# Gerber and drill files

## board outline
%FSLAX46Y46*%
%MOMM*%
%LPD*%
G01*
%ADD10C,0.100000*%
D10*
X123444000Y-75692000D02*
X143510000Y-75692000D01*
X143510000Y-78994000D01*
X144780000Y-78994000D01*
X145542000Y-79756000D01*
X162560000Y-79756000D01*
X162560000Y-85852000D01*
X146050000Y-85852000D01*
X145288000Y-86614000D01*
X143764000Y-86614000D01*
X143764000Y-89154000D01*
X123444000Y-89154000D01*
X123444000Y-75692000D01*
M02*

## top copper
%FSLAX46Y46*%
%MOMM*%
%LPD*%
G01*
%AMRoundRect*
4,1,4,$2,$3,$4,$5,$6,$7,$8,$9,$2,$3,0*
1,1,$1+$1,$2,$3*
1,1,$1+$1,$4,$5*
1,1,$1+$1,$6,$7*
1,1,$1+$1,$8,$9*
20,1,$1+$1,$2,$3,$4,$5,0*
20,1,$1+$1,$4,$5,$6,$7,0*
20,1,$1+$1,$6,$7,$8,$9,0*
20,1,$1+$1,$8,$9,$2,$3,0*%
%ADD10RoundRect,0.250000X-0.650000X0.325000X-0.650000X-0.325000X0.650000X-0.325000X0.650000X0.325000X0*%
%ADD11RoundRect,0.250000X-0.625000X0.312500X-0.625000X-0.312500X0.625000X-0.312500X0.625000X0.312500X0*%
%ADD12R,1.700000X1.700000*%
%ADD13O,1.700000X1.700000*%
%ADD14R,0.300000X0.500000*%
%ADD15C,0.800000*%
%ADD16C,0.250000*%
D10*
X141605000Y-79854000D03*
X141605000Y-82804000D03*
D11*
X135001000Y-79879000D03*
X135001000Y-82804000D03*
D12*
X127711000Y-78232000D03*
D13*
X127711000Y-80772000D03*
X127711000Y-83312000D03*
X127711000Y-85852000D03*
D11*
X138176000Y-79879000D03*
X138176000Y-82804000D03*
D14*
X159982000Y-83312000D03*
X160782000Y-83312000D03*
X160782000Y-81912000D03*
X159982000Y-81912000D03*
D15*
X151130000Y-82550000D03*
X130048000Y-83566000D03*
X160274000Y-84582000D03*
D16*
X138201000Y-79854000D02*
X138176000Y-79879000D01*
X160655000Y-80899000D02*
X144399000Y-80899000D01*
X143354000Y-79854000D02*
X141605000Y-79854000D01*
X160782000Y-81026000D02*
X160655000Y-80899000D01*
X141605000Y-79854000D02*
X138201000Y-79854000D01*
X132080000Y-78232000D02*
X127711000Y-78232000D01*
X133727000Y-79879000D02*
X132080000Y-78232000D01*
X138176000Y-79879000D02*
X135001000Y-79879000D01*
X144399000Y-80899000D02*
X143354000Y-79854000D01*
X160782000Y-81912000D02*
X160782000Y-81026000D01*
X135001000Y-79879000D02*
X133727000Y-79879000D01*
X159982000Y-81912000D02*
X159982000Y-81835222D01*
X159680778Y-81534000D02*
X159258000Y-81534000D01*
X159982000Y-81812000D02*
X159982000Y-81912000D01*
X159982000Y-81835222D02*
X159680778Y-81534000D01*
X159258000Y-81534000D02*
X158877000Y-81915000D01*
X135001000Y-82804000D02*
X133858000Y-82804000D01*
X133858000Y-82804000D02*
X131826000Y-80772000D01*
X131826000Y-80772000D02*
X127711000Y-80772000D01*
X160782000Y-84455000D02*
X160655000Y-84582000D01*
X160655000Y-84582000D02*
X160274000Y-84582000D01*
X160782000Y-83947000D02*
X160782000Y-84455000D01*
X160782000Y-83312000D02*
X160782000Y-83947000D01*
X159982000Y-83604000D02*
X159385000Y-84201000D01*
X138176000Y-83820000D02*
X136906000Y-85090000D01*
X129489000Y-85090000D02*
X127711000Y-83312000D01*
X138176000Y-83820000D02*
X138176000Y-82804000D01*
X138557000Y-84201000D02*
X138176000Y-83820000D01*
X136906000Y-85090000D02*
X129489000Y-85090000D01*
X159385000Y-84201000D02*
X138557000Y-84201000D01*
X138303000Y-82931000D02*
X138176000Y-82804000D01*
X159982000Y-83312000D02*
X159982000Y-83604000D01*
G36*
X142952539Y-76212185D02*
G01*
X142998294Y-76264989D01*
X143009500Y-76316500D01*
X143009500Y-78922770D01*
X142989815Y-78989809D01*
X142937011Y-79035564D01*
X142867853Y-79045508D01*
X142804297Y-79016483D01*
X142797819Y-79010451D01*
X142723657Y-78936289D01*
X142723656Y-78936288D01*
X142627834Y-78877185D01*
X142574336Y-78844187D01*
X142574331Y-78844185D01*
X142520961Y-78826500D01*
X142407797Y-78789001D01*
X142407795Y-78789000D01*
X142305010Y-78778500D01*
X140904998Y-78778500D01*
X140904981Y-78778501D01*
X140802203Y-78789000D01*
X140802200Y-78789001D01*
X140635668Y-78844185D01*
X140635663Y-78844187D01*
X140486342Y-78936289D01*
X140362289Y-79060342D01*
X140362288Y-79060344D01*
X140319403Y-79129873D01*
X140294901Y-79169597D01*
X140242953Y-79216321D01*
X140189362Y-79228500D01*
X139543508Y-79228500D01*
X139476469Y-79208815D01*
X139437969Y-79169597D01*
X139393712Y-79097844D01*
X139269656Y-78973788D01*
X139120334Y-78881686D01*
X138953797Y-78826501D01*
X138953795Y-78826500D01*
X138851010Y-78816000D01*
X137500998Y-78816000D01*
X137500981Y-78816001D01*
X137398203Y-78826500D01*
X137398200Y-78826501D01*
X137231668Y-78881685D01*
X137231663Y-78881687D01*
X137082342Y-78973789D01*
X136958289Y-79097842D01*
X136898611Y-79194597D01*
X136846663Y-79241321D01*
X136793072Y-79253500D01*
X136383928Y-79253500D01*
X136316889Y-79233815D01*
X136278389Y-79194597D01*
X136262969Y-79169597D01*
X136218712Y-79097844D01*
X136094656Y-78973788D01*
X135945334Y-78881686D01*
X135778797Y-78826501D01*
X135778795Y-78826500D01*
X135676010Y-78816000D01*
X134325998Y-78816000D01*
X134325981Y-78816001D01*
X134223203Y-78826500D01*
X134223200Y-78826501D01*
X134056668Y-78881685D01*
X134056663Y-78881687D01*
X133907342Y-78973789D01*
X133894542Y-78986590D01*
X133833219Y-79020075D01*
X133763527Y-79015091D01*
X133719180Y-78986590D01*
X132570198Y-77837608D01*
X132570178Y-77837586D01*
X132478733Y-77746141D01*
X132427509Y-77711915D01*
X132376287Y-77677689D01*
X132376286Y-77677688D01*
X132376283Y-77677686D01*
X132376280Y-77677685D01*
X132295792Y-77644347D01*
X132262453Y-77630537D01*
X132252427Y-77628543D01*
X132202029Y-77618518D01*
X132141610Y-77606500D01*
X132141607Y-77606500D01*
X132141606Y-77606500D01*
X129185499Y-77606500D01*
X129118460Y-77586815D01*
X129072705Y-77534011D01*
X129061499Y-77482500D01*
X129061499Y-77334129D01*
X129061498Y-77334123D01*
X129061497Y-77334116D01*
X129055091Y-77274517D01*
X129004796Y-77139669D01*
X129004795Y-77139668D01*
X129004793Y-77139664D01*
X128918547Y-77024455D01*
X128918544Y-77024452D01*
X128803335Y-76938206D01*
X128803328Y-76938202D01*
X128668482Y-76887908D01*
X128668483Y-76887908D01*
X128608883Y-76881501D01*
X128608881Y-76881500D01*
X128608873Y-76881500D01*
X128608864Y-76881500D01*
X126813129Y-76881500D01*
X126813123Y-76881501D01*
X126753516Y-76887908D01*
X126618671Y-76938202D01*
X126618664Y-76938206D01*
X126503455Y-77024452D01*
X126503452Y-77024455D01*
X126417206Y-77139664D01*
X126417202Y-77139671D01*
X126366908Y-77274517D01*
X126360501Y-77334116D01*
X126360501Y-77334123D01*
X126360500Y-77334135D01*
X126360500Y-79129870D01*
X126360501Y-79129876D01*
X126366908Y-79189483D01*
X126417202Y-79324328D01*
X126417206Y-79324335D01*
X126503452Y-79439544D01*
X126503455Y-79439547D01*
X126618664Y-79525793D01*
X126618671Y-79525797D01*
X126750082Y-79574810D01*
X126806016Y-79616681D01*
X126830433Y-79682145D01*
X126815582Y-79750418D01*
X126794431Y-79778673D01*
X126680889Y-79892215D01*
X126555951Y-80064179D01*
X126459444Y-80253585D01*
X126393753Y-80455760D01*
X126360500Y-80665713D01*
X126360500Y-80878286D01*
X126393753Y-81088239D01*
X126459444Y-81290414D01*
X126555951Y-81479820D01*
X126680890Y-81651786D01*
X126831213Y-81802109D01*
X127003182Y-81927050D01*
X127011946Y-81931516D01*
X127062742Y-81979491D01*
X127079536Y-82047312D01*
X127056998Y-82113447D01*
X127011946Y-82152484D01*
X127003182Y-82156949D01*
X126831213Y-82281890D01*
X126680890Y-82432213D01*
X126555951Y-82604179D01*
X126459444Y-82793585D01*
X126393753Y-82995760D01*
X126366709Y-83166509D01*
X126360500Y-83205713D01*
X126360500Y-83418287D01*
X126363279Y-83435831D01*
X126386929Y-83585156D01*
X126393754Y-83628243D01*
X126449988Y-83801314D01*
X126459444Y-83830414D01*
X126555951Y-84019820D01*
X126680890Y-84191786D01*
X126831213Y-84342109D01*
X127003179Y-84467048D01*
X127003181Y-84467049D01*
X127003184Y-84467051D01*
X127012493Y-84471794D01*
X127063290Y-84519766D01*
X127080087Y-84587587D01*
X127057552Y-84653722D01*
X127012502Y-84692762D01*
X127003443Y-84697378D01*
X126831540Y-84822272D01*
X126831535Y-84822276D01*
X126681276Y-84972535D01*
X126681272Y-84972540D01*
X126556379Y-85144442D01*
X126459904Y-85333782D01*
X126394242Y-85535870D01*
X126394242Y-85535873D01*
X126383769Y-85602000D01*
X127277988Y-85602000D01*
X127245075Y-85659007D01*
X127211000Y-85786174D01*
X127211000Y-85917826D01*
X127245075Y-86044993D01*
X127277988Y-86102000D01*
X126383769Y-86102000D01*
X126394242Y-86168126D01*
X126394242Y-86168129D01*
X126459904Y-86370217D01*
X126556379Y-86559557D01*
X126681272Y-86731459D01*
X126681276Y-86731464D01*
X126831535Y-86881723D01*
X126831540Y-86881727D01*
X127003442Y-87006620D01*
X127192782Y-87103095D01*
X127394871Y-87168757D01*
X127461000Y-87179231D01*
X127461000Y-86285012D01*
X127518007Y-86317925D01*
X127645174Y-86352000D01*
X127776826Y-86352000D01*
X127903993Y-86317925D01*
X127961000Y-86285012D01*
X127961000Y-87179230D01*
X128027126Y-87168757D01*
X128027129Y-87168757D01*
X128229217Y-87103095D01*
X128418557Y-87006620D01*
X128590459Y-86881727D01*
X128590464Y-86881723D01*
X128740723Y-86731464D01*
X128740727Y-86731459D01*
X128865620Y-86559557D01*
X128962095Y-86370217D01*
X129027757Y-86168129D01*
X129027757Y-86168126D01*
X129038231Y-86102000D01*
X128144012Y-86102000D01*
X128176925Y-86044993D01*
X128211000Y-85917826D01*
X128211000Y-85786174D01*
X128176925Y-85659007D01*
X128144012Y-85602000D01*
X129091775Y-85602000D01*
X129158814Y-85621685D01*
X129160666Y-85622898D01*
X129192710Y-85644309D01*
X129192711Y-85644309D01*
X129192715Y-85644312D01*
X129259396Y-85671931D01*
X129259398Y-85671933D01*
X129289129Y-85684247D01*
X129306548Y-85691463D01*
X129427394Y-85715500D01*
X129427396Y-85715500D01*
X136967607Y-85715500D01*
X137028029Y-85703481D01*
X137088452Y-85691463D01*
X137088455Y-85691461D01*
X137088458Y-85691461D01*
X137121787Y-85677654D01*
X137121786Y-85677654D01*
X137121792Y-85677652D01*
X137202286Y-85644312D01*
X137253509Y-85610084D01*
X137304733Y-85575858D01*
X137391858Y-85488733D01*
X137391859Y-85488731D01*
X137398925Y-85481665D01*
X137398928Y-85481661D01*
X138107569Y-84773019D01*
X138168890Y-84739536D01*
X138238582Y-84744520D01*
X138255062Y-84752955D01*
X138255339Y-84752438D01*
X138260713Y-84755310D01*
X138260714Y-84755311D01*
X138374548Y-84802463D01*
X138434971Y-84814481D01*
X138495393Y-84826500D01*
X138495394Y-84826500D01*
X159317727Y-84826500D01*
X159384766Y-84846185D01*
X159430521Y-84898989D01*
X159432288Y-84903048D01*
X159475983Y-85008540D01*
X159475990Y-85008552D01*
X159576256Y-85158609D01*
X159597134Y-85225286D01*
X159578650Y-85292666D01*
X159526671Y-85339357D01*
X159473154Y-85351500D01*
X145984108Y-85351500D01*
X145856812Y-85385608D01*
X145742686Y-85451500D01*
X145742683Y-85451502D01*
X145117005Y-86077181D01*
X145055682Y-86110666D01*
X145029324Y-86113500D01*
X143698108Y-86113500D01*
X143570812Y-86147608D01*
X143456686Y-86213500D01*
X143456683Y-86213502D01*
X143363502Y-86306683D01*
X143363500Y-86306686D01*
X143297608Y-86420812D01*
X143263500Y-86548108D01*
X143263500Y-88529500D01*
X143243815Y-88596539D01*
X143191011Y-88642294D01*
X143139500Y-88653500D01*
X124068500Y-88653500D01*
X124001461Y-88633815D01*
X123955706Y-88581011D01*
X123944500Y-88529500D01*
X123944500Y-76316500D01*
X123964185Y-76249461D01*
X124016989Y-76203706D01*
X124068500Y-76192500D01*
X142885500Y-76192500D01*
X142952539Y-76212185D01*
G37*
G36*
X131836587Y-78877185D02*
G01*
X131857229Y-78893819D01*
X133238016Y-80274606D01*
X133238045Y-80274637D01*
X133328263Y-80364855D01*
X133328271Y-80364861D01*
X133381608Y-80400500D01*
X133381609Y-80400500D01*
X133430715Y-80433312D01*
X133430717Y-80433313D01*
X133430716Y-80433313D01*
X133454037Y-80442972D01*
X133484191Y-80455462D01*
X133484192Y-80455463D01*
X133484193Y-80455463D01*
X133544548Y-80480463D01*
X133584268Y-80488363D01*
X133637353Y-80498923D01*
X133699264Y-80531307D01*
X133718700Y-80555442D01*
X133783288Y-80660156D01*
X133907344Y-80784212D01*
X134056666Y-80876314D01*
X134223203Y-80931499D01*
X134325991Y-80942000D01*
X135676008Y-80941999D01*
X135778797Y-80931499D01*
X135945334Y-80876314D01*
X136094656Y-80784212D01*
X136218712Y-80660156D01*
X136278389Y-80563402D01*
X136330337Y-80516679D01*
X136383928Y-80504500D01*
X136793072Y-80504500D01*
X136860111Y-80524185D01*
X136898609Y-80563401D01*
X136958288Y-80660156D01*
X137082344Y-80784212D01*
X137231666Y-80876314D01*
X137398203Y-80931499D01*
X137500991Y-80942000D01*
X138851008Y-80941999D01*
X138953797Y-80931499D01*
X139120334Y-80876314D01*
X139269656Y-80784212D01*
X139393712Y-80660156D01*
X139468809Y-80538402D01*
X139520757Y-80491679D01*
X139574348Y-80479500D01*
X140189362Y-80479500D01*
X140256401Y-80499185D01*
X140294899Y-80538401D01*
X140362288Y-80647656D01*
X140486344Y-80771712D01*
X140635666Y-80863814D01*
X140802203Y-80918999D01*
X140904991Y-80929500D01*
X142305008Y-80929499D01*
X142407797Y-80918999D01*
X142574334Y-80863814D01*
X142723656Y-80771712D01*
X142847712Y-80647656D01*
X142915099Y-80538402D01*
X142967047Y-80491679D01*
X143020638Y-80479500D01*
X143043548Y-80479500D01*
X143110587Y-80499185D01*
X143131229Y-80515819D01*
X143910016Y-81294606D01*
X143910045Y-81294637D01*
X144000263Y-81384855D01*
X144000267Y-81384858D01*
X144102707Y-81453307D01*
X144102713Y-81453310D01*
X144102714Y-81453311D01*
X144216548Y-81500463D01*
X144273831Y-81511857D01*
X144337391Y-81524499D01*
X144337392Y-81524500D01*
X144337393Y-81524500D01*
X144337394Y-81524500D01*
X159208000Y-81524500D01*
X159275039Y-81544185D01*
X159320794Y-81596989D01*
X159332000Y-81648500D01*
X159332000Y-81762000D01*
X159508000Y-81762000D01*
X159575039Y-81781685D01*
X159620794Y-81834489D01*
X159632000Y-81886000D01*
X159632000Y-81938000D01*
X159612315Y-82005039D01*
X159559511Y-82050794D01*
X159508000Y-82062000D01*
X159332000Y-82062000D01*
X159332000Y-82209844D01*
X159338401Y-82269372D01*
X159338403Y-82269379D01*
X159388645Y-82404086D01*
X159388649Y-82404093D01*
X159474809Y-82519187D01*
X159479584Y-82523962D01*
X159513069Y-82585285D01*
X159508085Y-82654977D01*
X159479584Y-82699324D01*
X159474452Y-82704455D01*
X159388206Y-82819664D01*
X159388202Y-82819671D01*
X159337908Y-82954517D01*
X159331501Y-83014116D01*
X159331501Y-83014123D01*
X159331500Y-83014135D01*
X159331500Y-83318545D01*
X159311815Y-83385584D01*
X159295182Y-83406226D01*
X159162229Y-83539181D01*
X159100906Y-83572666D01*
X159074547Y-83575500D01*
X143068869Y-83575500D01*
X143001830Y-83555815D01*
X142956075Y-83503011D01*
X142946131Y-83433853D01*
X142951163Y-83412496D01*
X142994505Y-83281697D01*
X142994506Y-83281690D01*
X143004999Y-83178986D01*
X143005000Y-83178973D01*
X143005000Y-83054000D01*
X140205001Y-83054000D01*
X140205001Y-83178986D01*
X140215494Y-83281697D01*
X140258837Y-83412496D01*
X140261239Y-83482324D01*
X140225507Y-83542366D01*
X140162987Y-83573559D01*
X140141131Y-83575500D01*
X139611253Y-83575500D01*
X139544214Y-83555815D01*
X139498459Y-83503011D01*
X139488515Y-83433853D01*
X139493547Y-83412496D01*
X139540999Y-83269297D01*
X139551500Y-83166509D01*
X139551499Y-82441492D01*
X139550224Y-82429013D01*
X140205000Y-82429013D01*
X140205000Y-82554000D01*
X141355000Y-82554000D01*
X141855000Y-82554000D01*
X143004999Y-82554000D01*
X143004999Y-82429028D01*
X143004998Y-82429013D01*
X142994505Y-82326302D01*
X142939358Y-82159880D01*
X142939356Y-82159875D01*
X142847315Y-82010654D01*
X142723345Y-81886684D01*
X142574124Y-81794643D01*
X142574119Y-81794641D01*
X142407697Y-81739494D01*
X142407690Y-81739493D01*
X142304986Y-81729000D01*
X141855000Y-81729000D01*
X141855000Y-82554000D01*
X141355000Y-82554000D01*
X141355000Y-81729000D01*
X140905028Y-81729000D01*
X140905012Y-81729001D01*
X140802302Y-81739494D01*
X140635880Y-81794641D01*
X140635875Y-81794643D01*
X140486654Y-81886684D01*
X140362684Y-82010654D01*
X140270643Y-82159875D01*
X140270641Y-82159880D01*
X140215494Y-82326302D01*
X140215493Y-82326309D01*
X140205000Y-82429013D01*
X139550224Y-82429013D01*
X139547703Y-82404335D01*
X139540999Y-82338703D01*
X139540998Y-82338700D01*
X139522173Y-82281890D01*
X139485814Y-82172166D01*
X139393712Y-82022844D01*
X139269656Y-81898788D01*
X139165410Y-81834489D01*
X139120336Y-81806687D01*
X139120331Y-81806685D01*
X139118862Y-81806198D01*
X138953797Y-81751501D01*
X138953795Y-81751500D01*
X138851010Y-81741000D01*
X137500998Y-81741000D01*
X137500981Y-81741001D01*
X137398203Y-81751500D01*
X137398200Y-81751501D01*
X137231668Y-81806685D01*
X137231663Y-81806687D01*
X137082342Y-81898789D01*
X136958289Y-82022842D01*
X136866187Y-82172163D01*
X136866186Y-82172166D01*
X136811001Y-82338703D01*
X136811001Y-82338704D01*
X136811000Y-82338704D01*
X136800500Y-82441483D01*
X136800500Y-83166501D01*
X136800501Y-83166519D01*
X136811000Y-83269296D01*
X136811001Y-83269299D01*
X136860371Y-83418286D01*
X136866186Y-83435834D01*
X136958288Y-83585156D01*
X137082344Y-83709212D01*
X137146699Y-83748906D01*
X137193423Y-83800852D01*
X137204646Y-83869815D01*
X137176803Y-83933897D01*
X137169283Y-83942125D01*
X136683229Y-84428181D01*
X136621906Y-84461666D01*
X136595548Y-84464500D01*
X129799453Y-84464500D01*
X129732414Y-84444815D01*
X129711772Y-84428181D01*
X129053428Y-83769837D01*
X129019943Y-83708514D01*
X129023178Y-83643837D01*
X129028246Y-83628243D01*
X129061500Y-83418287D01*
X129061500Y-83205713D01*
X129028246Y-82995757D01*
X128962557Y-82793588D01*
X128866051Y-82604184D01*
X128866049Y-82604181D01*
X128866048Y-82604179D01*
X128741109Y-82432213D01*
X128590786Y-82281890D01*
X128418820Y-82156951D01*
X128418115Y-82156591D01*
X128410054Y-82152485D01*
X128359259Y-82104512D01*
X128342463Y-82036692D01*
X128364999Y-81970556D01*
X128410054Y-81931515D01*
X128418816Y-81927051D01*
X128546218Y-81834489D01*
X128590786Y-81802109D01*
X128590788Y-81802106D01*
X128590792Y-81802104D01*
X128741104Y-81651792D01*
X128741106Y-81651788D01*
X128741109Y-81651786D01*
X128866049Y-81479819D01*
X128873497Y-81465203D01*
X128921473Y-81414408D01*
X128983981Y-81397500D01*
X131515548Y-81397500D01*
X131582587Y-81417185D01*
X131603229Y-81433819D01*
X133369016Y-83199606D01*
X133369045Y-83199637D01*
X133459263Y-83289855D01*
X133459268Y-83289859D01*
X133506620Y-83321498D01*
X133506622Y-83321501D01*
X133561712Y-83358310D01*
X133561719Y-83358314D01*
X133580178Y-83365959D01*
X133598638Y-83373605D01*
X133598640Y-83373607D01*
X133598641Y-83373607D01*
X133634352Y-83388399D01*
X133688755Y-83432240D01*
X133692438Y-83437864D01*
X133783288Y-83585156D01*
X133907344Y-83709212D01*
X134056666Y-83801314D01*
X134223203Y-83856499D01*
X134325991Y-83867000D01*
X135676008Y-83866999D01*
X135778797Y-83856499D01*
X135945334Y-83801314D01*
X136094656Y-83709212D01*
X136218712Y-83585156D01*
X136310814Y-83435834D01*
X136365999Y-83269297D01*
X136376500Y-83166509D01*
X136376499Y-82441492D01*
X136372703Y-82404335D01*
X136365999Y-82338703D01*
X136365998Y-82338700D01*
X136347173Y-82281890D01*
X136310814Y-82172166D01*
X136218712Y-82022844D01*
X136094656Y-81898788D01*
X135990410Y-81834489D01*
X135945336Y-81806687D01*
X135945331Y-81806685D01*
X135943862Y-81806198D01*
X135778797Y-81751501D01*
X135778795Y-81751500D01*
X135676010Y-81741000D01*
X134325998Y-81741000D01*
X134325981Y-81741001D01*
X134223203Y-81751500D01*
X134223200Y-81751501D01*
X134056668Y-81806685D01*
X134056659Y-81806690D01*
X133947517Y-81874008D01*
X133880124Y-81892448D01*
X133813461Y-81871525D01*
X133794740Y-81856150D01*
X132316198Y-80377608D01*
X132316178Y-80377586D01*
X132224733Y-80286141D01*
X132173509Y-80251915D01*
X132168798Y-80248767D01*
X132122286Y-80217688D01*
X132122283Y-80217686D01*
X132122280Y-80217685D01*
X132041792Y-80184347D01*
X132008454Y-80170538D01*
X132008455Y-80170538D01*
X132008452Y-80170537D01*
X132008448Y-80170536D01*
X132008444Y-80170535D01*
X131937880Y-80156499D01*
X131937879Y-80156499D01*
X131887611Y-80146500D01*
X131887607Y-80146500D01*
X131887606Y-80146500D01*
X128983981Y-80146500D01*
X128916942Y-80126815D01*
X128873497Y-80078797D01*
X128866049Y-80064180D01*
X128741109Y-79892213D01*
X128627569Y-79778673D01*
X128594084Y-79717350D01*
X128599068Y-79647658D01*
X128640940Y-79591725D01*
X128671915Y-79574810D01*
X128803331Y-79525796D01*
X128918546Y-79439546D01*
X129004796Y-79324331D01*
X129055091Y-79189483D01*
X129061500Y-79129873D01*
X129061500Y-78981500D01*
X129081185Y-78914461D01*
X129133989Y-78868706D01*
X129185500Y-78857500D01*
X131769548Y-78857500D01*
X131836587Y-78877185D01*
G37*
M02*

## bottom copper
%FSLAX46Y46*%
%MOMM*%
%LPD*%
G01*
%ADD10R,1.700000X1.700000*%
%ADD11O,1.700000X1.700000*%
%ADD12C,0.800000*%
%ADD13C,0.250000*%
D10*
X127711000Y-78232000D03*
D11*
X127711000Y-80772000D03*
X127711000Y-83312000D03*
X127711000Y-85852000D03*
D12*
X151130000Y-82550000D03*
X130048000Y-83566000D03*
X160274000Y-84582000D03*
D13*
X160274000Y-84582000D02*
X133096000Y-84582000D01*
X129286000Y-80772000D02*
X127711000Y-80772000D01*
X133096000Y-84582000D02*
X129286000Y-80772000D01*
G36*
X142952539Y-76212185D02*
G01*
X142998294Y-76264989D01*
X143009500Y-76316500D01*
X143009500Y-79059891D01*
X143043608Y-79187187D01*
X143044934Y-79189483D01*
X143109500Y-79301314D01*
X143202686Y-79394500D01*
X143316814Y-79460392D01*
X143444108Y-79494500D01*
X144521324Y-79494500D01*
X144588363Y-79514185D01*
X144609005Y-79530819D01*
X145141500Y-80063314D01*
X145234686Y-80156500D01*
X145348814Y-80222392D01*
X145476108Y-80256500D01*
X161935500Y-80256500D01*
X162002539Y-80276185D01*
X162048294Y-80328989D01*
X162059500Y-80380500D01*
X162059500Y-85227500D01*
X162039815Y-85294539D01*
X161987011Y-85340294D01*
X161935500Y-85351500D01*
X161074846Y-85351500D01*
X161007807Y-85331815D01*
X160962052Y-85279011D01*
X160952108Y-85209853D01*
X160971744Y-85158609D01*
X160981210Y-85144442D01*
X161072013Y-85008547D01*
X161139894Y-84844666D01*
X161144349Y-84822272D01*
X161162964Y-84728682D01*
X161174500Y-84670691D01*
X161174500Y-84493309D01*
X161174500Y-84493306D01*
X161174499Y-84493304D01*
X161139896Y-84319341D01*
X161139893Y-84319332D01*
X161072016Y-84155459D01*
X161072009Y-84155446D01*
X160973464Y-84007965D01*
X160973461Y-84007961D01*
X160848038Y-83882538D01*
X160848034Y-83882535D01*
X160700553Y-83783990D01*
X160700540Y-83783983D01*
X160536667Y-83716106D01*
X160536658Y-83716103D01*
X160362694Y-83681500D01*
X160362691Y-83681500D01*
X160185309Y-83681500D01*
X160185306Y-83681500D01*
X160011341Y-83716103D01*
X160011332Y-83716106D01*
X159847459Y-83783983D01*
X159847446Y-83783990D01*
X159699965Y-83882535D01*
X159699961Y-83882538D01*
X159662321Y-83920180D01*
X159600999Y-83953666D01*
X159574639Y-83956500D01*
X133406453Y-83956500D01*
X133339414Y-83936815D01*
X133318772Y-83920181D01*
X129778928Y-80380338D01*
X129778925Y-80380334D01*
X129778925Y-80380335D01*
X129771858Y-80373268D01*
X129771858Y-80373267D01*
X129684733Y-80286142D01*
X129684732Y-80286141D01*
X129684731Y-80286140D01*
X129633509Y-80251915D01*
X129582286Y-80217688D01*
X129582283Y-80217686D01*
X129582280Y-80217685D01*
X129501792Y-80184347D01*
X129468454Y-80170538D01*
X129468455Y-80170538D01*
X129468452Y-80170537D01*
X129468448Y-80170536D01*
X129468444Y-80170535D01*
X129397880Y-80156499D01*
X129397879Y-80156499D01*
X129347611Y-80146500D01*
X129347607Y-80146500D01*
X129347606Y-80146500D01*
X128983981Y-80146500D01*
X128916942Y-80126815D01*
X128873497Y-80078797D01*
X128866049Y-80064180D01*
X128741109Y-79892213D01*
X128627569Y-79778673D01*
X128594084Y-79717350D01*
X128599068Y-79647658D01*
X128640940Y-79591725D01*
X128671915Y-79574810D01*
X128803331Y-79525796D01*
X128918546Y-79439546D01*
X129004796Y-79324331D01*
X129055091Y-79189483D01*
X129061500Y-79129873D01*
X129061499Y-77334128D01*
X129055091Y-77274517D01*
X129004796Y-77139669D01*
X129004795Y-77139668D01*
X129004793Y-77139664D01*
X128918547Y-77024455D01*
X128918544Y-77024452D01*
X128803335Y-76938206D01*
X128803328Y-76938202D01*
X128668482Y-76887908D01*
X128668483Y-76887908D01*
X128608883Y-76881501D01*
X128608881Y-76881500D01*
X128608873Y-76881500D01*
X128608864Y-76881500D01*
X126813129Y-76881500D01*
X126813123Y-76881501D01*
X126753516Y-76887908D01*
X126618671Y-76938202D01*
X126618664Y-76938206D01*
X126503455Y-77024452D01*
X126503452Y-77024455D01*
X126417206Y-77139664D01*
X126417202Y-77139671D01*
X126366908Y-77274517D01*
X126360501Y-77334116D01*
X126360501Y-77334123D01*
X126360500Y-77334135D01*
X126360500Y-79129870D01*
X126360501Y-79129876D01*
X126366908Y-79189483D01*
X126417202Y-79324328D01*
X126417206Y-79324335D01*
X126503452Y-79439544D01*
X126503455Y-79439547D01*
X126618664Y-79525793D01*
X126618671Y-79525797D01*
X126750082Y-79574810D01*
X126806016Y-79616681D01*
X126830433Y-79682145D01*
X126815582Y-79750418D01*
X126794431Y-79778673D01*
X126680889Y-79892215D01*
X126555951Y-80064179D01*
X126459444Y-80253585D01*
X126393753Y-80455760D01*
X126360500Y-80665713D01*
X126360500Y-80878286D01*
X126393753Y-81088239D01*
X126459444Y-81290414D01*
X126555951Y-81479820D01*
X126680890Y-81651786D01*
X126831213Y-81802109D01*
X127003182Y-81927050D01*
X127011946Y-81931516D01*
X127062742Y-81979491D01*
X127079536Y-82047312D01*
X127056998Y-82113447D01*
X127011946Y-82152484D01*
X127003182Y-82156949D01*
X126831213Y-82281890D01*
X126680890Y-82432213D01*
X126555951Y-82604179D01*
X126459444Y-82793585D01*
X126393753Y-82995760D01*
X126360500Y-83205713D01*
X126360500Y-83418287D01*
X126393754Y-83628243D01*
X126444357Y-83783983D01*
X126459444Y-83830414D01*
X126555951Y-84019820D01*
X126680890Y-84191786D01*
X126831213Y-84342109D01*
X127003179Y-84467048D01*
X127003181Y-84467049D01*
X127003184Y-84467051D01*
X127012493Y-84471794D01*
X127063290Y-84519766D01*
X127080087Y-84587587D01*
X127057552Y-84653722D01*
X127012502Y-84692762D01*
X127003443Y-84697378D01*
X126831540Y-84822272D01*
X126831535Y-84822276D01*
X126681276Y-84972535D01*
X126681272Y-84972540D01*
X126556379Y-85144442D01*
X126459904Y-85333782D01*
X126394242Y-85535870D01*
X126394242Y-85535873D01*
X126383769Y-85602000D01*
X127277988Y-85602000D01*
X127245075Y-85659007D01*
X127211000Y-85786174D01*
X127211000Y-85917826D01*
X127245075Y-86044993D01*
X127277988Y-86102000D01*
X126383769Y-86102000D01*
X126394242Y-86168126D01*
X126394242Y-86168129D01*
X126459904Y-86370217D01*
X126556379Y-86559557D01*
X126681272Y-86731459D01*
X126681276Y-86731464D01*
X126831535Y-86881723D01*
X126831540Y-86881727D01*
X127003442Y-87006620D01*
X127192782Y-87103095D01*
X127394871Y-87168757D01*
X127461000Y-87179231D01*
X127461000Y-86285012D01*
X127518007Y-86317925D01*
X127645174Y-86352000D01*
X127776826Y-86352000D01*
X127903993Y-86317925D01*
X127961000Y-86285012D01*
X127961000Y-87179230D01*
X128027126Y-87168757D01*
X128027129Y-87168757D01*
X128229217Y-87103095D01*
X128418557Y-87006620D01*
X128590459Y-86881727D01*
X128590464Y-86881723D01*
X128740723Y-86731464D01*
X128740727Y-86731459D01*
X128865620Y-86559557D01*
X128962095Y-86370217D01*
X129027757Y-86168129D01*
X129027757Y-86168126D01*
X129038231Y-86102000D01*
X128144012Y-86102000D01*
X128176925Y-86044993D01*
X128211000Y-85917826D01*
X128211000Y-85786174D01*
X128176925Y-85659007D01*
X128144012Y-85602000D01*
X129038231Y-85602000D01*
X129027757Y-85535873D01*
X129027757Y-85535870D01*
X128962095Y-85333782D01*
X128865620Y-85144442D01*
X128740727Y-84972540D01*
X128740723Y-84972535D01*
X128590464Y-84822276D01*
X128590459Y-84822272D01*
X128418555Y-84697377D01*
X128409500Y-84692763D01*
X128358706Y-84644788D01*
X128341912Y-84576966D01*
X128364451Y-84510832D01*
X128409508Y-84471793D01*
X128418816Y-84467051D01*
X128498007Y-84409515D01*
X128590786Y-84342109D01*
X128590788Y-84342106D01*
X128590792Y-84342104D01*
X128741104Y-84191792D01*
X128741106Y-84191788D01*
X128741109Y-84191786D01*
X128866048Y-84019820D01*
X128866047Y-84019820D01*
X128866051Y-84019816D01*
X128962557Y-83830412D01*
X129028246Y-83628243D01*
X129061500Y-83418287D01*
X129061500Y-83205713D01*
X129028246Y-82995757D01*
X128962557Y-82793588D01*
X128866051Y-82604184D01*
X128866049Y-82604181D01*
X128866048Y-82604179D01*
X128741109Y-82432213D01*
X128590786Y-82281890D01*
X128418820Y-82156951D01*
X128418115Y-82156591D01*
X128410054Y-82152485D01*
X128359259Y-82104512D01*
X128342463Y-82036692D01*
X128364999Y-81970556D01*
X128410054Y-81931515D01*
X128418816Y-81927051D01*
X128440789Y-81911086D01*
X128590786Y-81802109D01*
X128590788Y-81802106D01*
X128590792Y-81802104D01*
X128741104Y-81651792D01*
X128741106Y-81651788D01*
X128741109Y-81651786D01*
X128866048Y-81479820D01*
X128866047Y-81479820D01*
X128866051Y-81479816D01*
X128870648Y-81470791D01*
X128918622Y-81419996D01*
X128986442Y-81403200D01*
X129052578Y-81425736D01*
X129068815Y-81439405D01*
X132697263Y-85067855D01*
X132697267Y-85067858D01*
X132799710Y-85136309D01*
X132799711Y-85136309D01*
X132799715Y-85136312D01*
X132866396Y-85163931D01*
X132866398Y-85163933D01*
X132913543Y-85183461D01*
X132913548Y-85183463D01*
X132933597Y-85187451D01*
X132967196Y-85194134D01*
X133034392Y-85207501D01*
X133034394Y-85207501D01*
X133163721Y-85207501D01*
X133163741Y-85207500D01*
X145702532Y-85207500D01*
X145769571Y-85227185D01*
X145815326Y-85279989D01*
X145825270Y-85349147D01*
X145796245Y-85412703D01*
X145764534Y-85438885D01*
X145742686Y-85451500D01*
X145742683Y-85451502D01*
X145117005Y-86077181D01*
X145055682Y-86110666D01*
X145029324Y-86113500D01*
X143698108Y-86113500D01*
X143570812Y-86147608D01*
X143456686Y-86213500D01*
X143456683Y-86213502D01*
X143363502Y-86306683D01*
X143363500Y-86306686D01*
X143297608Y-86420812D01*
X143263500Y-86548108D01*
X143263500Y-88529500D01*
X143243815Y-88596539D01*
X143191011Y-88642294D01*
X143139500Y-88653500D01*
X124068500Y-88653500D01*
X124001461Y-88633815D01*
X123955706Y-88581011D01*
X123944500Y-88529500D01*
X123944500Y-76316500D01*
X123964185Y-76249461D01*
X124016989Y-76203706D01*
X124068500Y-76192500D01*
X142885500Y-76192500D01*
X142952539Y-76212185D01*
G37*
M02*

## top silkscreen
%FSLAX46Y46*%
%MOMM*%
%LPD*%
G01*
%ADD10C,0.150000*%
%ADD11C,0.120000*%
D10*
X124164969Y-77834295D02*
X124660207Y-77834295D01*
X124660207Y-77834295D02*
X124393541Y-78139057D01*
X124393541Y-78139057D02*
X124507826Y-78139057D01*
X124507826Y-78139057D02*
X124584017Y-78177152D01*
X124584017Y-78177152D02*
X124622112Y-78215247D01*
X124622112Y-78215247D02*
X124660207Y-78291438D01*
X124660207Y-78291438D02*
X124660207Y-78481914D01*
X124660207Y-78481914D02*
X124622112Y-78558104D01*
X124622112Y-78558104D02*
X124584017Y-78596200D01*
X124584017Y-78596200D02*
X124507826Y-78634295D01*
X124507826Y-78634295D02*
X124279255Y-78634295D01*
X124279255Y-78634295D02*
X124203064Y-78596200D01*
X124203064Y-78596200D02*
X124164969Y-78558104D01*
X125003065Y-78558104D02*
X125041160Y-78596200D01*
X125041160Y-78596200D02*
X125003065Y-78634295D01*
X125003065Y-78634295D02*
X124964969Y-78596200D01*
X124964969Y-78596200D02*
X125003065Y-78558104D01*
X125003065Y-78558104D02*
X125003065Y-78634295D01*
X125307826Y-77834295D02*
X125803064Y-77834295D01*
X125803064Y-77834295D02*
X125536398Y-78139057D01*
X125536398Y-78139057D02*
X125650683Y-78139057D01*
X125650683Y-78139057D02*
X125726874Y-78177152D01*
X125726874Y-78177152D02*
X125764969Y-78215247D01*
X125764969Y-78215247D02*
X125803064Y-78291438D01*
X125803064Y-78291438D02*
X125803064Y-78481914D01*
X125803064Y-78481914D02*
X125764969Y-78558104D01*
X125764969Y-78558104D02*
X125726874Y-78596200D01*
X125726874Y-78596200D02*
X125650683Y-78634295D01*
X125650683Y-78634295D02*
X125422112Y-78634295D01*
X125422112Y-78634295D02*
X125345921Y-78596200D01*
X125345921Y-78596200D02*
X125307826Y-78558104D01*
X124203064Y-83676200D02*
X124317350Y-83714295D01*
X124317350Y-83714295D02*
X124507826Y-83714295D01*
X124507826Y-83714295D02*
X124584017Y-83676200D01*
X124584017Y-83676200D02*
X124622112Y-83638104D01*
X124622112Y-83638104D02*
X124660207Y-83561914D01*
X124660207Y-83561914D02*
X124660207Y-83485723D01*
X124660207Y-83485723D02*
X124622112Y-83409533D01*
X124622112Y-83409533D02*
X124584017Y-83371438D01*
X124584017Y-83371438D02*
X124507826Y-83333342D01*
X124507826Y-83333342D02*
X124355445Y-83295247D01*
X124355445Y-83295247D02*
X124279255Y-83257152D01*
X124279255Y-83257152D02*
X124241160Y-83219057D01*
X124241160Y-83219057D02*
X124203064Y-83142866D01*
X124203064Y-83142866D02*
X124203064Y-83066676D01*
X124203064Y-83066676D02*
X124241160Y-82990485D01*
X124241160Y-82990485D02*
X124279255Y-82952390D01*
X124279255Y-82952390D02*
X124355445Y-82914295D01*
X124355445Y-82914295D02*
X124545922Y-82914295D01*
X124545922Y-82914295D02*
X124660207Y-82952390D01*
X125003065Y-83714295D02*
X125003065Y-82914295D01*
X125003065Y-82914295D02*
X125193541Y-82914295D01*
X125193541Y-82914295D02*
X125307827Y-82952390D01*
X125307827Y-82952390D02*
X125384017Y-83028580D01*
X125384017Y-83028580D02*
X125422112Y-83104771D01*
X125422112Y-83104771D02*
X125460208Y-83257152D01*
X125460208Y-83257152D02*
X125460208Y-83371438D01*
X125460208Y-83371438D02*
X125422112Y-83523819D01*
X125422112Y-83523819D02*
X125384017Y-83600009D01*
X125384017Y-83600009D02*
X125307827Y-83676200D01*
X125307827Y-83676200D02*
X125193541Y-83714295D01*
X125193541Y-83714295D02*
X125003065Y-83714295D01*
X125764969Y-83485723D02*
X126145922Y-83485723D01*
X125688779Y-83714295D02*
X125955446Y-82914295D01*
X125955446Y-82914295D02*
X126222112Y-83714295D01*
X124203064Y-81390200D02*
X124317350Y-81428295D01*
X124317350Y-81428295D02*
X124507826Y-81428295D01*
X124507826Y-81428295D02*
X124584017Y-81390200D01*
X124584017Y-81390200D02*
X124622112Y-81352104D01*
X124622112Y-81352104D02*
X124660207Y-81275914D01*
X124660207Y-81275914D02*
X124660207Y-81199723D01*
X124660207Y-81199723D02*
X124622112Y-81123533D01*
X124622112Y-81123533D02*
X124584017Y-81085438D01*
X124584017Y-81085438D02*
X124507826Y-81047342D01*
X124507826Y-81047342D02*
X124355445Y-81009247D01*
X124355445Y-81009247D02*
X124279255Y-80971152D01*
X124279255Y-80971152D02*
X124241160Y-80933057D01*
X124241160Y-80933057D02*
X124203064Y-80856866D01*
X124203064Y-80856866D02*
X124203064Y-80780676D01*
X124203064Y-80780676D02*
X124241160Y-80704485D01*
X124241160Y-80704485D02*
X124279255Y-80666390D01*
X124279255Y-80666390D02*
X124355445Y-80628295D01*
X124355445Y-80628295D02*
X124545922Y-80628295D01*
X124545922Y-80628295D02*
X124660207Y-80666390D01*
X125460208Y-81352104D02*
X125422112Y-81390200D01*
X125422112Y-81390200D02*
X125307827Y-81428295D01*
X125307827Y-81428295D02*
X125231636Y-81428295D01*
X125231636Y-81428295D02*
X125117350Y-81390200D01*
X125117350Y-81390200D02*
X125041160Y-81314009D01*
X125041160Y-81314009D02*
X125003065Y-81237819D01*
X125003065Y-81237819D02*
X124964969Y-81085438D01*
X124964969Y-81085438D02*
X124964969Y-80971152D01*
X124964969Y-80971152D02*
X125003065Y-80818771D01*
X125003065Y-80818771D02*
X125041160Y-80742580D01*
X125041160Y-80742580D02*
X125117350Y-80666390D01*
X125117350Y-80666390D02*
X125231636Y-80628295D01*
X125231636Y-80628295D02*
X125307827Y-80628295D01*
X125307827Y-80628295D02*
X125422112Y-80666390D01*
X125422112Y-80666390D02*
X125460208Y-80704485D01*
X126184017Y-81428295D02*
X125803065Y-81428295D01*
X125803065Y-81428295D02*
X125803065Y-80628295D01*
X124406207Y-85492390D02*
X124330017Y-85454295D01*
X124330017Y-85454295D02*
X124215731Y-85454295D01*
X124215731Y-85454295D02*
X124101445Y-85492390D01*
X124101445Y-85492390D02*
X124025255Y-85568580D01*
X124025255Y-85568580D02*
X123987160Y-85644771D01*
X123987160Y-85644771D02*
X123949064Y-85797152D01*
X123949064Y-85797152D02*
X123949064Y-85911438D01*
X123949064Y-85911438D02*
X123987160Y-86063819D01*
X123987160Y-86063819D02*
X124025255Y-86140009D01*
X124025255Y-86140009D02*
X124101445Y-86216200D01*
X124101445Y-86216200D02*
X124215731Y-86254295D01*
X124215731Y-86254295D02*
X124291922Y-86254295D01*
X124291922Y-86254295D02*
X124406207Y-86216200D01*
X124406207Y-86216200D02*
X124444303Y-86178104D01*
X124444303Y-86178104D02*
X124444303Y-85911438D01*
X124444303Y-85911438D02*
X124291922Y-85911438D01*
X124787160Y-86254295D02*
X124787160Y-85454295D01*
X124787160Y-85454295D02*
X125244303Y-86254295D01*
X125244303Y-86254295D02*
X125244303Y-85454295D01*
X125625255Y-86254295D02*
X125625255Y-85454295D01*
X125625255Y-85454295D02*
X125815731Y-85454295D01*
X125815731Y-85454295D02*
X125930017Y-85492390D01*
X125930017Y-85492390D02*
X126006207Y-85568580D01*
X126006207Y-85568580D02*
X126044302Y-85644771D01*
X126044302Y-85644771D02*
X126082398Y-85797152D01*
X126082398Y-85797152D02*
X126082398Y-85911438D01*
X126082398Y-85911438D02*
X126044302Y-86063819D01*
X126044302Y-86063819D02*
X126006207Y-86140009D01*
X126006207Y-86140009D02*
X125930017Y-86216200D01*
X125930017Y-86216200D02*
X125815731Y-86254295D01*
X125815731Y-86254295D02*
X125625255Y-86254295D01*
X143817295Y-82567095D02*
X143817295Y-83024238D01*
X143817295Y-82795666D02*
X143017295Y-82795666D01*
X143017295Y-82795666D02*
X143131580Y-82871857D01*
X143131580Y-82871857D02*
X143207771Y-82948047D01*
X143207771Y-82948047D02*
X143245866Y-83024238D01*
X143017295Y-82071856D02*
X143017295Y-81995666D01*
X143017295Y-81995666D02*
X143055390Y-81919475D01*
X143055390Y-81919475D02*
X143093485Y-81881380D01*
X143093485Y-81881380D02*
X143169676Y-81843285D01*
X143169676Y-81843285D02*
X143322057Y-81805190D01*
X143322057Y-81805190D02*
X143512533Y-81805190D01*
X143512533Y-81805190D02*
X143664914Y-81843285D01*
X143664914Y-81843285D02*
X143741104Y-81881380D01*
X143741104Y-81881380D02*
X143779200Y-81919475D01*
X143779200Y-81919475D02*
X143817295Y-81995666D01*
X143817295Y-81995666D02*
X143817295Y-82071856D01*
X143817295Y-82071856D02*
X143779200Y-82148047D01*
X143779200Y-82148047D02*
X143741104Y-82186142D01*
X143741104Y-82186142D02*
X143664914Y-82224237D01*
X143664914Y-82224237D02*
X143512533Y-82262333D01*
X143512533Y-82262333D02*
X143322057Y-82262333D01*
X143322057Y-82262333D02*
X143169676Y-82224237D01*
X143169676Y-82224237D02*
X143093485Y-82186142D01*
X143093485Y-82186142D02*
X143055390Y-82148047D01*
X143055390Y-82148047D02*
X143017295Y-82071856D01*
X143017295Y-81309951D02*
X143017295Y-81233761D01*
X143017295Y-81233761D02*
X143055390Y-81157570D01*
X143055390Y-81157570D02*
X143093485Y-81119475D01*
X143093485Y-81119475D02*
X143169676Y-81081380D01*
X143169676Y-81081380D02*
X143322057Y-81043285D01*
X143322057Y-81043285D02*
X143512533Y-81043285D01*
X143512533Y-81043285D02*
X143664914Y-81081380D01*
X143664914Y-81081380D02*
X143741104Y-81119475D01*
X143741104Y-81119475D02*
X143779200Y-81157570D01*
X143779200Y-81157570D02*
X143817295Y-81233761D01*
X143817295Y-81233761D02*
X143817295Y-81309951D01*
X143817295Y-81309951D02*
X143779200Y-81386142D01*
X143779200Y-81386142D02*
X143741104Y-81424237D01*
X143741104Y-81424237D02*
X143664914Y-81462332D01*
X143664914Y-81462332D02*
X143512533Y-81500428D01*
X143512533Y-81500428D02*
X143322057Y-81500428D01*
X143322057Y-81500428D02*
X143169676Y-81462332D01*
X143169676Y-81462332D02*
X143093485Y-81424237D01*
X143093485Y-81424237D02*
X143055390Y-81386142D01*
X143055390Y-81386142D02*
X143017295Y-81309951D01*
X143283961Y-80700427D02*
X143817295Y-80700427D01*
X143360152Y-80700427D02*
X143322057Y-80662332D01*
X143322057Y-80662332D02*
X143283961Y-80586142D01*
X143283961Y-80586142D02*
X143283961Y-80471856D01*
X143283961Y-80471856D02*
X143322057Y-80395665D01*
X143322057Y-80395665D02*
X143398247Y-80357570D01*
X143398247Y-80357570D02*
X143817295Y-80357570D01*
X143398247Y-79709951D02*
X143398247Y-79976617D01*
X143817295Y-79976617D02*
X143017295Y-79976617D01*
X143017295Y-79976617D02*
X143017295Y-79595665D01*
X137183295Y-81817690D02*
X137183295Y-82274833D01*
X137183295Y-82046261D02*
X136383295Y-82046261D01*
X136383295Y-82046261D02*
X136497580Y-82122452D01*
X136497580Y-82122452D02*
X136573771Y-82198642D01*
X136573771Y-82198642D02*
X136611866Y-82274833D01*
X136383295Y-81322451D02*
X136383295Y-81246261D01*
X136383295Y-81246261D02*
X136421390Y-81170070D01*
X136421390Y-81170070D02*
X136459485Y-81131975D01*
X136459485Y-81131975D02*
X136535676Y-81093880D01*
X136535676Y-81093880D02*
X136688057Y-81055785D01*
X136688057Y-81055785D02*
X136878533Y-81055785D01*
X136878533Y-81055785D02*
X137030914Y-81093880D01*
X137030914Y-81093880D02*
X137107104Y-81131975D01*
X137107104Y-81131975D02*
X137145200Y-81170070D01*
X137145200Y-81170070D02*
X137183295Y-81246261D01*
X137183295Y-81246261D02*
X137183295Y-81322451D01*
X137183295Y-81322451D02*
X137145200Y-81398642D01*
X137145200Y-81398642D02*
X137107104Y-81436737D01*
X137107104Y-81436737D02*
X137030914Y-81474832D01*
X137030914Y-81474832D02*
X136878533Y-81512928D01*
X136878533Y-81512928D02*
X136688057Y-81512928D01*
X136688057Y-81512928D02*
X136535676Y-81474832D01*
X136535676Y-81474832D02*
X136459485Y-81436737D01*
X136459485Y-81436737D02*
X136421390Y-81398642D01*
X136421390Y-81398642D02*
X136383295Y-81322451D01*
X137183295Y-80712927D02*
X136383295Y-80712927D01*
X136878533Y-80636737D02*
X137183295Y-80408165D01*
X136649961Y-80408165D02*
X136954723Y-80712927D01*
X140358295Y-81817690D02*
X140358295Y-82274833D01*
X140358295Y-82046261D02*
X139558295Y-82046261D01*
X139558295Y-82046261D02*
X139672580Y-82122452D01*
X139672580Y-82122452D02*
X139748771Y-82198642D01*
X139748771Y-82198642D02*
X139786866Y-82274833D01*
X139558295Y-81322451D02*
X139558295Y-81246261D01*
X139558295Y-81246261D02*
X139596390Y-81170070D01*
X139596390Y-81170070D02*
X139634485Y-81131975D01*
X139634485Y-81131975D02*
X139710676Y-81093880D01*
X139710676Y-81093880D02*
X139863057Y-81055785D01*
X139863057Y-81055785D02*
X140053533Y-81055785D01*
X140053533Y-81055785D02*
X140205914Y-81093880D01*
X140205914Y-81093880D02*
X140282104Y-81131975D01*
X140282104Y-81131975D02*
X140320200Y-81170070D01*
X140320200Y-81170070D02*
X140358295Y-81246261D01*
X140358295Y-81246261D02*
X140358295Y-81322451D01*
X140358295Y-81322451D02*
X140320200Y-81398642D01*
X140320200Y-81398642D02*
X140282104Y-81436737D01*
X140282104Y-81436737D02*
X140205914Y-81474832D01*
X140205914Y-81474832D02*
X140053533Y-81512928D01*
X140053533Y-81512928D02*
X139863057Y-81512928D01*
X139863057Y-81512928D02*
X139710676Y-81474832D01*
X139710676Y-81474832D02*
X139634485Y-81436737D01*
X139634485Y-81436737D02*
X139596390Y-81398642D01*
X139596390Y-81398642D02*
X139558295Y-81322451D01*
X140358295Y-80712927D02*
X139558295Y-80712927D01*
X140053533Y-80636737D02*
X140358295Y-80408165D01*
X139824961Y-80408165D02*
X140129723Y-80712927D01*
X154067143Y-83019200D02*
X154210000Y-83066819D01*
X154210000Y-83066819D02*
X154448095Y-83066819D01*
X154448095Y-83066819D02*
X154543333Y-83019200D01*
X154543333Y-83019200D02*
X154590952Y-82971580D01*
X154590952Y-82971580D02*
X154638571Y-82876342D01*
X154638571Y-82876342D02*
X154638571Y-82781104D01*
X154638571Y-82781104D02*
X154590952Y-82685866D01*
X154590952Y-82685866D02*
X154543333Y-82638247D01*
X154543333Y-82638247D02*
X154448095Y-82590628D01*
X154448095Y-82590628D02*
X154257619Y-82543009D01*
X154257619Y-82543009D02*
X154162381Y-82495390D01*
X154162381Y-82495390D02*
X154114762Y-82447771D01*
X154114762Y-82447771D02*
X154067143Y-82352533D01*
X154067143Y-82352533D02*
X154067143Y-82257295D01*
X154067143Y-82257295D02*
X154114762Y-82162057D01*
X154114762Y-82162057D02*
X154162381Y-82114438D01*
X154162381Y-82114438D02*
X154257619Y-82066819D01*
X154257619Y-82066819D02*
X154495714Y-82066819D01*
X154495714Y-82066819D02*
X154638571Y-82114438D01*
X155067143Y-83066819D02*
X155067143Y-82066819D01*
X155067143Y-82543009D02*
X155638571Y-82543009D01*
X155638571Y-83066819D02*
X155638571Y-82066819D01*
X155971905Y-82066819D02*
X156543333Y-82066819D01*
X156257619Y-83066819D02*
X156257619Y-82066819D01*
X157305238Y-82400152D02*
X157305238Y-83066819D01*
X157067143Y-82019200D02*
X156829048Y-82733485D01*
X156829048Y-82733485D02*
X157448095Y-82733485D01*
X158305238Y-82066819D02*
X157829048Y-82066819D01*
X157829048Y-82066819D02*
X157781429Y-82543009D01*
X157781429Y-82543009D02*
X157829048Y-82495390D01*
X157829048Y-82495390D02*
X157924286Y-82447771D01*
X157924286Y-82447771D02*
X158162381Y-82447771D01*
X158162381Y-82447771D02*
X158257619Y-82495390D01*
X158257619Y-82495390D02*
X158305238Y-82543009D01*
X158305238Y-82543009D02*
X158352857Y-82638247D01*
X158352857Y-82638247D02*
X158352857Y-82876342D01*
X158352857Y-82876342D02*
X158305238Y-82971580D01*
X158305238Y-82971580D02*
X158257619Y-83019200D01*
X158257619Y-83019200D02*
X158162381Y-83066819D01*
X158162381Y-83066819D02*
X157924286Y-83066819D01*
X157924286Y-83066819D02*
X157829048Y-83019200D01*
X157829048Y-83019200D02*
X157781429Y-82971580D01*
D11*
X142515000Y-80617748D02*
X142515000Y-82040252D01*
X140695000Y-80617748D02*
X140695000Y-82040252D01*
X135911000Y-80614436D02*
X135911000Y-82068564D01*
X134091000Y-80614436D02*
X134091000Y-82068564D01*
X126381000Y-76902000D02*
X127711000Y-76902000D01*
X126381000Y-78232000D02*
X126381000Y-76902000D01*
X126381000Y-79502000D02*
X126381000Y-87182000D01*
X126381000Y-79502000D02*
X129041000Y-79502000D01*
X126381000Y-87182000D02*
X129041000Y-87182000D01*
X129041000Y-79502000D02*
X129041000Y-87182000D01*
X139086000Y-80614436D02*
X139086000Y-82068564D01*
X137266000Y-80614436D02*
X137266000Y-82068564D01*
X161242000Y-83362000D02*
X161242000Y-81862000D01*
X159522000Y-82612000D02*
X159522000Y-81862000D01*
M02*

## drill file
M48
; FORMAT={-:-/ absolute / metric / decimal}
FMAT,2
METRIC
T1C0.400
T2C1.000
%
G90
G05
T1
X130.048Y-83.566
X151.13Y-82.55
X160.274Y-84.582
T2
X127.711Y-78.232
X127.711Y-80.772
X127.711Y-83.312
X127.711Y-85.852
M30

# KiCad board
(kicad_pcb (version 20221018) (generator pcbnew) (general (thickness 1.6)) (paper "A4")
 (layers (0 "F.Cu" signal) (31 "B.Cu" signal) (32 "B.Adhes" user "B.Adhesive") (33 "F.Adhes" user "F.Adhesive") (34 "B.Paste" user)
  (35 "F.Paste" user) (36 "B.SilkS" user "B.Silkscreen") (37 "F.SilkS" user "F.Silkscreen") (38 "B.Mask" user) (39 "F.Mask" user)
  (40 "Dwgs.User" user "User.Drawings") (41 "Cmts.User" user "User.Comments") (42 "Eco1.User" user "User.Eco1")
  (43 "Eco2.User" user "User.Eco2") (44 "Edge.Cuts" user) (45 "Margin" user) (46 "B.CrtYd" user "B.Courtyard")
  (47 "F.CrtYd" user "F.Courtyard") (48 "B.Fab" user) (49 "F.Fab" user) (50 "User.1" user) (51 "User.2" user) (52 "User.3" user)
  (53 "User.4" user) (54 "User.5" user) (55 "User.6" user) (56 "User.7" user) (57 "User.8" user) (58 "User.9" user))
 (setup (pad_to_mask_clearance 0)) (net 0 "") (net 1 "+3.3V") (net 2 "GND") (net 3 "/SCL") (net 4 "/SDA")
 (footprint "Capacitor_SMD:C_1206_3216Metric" (layer "F.Cu") (at 141.605 81.329 -90)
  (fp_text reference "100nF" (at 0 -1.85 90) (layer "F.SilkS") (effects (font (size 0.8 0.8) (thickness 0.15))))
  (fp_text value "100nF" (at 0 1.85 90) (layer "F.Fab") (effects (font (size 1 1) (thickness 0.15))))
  (fp_line (start -0.711252 -0.91) (end 0.711252 -0.91) (stroke (width 0.12) (type solid)) (layer "F.SilkS"))
  (fp_line (start -0.711252 0.91) (end 0.711252 0.91) (stroke (width 0.12) (type solid)) (layer "F.SilkS"))
  (pad "1" smd roundrect (at -1.475 0 270) (size 1.15 1.8) (layers "F.Cu" "F.Paste" "F.Mask") (roundrect_rratio 0.2173913043)
   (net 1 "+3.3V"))
  (pad "2" smd roundrect (at 1.475 0 270) (size 1.15 1.8) (layers "F.Cu" "F.Paste" "F.Mask") (roundrect_rratio 0.2173913043) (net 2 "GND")))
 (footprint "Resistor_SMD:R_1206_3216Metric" (layer "F.Cu") (at 135.001 81.3415 -90)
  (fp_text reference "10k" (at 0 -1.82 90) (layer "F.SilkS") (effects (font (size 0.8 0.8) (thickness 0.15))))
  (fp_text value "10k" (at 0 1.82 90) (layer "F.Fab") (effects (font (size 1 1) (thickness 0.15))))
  (fp_line (start -0.727064 -0.91) (end 0.727064 -0.91) (stroke (width 0.12) (type solid)) (layer "F.SilkS"))
  (fp_line (start -0.727064 0.91) (end 0.727064 0.91) (stroke (width 0.12) (type solid)) (layer "F.SilkS"))
  (pad "1" smd roundrect (at -1.4625 0 270) (size 1.125 1.75) (layers "F.Cu" "F.Paste" "F.Mask") (roundrect_rratio 0.2222222222)
   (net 1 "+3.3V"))
  (pad "2" smd roundrect (at 1.4625 0 270) (size 1.125 1.75) (layers "F.Cu" "F.Paste" "F.Mask") (roundrect_rratio 0.2222222222)
   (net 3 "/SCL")))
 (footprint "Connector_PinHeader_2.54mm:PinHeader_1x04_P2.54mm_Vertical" (layer "F.Cu") (at 127.711 78.232)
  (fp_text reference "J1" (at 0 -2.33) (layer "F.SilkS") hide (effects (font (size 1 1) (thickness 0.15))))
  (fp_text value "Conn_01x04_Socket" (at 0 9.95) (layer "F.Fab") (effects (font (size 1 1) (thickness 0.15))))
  (fp_line (start -1.33 -1.33) (end 0 -1.33) (stroke (width 0.12) (type solid)) (layer "F.SilkS"))
  (fp_line (start -1.33 0) (end -1.33 -1.33) (stroke (width 0.12) (type solid)) (layer "F.SilkS"))
  (fp_line (start -1.33 1.27) (end -1.33 8.95) (stroke (width 0.12) (type solid)) (layer "F.SilkS"))
  (fp_line (start -1.33 1.27) (end 1.33 1.27) (stroke (width 0.12) (type solid)) (layer "F.SilkS"))
  (fp_line (start -1.33 8.95) (end 1.33 8.95) (stroke (width 0.12) (type solid)) (layer "F.SilkS"))
  (fp_line (start 1.33 1.27) (end 1.33 8.95) (stroke (width 0.12) (type solid)) (layer "F.SilkS"))
  (pad "1" thru_hole rect (at 0 0) (size 1.7 1.7) (drill 1) (layers "*.Cu" "*.Mask") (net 1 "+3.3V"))
  (pad "2" thru_hole oval (at 0 2.54) (size 1.7 1.7) (drill 1) (layers "*.Cu" "*.Mask") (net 3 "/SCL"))
  (pad "3" thru_hole oval (at 0 5.08) (size 1.7 1.7) (drill 1) (layers "*.Cu" "*.Mask") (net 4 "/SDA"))
  (pad "4" thru_hole oval (at 0 7.62) (size 1.7 1.7) (drill 1) (layers "*.Cu" "*.Mask") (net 2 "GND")))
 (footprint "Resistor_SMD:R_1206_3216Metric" (layer "F.Cu") (at 138.176 81.3415 -90)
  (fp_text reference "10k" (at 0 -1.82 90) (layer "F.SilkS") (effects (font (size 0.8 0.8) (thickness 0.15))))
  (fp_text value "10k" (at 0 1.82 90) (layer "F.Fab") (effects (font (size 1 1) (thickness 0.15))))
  (fp_line (start -0.727064 -0.91) (end 0.727064 -0.91) (stroke (width 0.12) (type solid)) (layer "F.SilkS"))
  (fp_line (start -0.727064 0.91) (end 0.727064 0.91) (stroke (width 0.12) (type solid)) (layer "F.SilkS"))
  (pad "1" smd roundrect (at -1.4625 0 270) (size 1.125 1.75) (layers "F.Cu" "F.Paste" "F.Mask") (roundrect_rratio 0.2222222222)
   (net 1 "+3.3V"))
  (pad "2" smd roundrect (at 1.4625 0 270) (size 1.125 1.75) (layers "F.Cu" "F.Paste" "F.Mask") (roundrect_rratio 0.2222222222)
   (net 4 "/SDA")))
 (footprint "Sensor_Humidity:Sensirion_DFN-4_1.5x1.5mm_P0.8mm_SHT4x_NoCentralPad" (layer "F.Cu") (at 160.382 82.612 90)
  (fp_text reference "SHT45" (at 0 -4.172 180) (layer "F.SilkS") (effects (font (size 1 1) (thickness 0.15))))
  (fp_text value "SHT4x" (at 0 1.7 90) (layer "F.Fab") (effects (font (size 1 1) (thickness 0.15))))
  (fp_line (start -0.75 0.86) (end 0.75 0.86) (stroke (width 0.12) (type solid)) (layer "F.SilkS"))
  (fp_line (start 0 -0.86) (end 0.75 -0.86) (stroke (width 0.12) (type solid)) (layer "F.SilkS"))
  (pad "1" smd rect (at -0.7 -0.4 90) (size 0.5 0.3) (layers "F.Cu" "F.Paste" "F.Mask") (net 4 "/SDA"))
  (pad "2" smd rect (at -0.7 0.4 90) (size 0.5 0.3) (layers "F.Cu" "F.Paste" "F.Mask") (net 3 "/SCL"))
  (pad "3" smd rect (at 0.7 0.4 90) (size 0.5 0.3) (layers "F.Cu" "F.Paste" "F.Mask") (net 1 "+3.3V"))
  (pad "4" smd rect (at 0.7 -0.4 90) (size 0.5 0.3) (layers "F.Cu" "F.Paste" "F.Mask") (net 2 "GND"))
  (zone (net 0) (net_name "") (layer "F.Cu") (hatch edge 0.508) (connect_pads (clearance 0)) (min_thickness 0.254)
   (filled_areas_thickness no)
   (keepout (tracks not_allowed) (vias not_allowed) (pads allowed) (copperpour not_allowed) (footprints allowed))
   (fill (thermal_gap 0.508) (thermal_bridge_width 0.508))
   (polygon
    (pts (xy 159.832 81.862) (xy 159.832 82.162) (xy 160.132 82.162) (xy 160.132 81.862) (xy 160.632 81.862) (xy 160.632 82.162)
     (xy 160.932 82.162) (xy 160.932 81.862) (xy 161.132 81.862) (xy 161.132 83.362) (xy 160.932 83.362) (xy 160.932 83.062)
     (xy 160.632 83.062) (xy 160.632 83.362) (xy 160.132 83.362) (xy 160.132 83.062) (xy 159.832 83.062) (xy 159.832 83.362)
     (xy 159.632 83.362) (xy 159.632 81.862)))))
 (gr_poly
  (pts (xy 123.444 75.692) (xy 143.51 75.692) (xy 143.51 78.994) (xy 144.78 78.994) (xy 145.542 79.756) (xy 162.56 79.756)
   (xy 162.56 85.852) (xy 146.05 85.852) (xy 145.288 86.614) (xy 143.764 86.614) (xy 143.764 89.154) (xy 123.444 89.154))
  (stroke (width 0.1) (type solid)) (fill none) (layer "Edge.Cuts"))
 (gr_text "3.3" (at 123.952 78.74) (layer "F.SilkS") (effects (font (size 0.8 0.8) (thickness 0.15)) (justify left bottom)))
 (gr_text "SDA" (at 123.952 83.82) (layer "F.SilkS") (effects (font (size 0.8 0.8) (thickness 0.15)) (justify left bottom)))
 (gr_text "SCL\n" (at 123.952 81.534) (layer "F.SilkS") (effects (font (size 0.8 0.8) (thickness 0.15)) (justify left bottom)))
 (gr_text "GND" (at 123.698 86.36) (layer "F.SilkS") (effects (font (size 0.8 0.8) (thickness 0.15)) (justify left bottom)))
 (segment (start 138.201 79.854) (end 138.176 79.879) (width 0.25) (layer "F.Cu") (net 1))
 (segment (start 160.655 80.899) (end 144.399 80.899) (width 0.25) (layer "F.Cu") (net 1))
 (segment (start 143.354 79.854) (end 141.605 79.854) (width 0.25) (layer "F.Cu") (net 1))
 (segment (start 160.782 81.026) (end 160.655 80.899) (width 0.25) (layer "F.Cu") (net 1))
 (segment (start 141.605 79.854) (end 138.201 79.854) (width 0.25) (layer "F.Cu") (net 1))
 (segment (start 132.08 78.232) (end 127.711 78.232) (width 0.25) (layer "F.Cu") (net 1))
 (segment (start 133.727 79.879) (end 132.08 78.232) (width 0.25) (layer "F.Cu") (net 1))
 (segment (start 138.176 79.879) (end 135.001 79.879) (width 0.25) (layer "F.Cu") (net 1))
 (segment (start 144.399 80.899) (end 143.354 79.854) (width 0.25) (layer "F.Cu") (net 1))
 (segment (start 160.782 81.912) (end 160.782 81.026) (width 0.25) (layer "F.Cu") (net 1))
 (segment (start 135.001 79.879) (end 133.727 79.879) (width 0.25) (layer "F.Cu") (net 1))
 (segment (start 159.982 81.912) (end 159.982 81.835222) (width 0.25) (layer "F.Cu") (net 2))
 (segment (start 159.680778 81.534) (end 159.258 81.534) (width 0.25) (layer "F.Cu") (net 2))
 (segment (start 159.982 81.812) (end 159.982 81.912) (width 0.25) (layer "F.Cu") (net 2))
 (segment (start 159.982 81.835222) (end 159.680778 81.534) (width 0.25) (layer "F.Cu") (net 2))
 (segment (start 159.258 81.534) (end 158.877 81.915) (width 0.25) (layer "F.Cu") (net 2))
 (via (at 151.13 82.55) (size 0.8) (drill 0.4) (layers "F.Cu" "B.Cu") (free) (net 2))
 (via (at 130.048 83.566) (size 0.8) (drill 0.4) (layers "F.Cu" "B.Cu") (free) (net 2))
 (segment (start 135.001 82.804) (end 133.858 82.804) (width 0.25) (layer "F.Cu") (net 3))
 (segment (start 133.858 82.804) (end 131.826 80.772) (width 0.25) (layer "F.Cu") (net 3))
 (segment (start 131.826 80.772) (end 127.711 80.772) (width 0.25) (layer "F.Cu") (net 3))
 (segment (start 160.782 84.455) (end 160.655 84.582) (width 0.25) (layer "F.Cu") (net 3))
 (segment (start 160.655 84.582) (end 160.274 84.582) (width 0.25) (layer "F.Cu") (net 3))
 (segment (start 160.782 83.947) (end 160.782 84.455) (width 0.25) (layer "F.Cu") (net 3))
 (segment (start 160.782 83.312) (end 160.782 83.947) (width 0.25) (layer "F.Cu") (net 3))
 (via (at 160.274 84.582) (size 0.8) (drill 0.4) (layers "F.Cu" "B.Cu") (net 3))
 (segment (start 160.274 84.582) (end 133.096 84.582) (width 0.25) (layer "B.Cu") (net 3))
 (segment (start 129.286 80.772) (end 127.711 80.772) (width 0.25) (layer "B.Cu") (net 3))
 (segment (start 133.096 84.582) (end 129.286 80.772) (width 0.25) (layer "B.Cu") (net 3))
 (segment (start 159.982 83.604) (end 159.385 84.201) (width 0.25) (layer "F.Cu") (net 4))
 (segment (start 138.176 83.82) (end 136.906 85.09) (width 0.25) (layer "F.Cu") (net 4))
 (segment (start 129.489 85.09) (end 127.711 83.312) (width 0.25) (layer "F.Cu") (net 4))
 (segment (start 138.176 83.82) (end 138.176 82.804) (width 0.25) (layer "F.Cu") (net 4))
 (segment (start 138.557 84.201) (end 138.176 83.82) (width 0.25) (layer "F.Cu") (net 4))
 (segment (start 136.906 85.09) (end 129.489 85.09) (width 0.25) (layer "F.Cu") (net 4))
 (segment (start 159.385 84.201) (end 138.557 84.201) (width 0.25) (layer "F.Cu") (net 4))
 (segment (start 138.303 82.931) (end 138.176 82.804) (width 0.25) (layer "F.Cu") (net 4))
 (segment (start 159.982 83.312) (end 159.982 83.604) (width 0.25) (layer "F.Cu") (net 4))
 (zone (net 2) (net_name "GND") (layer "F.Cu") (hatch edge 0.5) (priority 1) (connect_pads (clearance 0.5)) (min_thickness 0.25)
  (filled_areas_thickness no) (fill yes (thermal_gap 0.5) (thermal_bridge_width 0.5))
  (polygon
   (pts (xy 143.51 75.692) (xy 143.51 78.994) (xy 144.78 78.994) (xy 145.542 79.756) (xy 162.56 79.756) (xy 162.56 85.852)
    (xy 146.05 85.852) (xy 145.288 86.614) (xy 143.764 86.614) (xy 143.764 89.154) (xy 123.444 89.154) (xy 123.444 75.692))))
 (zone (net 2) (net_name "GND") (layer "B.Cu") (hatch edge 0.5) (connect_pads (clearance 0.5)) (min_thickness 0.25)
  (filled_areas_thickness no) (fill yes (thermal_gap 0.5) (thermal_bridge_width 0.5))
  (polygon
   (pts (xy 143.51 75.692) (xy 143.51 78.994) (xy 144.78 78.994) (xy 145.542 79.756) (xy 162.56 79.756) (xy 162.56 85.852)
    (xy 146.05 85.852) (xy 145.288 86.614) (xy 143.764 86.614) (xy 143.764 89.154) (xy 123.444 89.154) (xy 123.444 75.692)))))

